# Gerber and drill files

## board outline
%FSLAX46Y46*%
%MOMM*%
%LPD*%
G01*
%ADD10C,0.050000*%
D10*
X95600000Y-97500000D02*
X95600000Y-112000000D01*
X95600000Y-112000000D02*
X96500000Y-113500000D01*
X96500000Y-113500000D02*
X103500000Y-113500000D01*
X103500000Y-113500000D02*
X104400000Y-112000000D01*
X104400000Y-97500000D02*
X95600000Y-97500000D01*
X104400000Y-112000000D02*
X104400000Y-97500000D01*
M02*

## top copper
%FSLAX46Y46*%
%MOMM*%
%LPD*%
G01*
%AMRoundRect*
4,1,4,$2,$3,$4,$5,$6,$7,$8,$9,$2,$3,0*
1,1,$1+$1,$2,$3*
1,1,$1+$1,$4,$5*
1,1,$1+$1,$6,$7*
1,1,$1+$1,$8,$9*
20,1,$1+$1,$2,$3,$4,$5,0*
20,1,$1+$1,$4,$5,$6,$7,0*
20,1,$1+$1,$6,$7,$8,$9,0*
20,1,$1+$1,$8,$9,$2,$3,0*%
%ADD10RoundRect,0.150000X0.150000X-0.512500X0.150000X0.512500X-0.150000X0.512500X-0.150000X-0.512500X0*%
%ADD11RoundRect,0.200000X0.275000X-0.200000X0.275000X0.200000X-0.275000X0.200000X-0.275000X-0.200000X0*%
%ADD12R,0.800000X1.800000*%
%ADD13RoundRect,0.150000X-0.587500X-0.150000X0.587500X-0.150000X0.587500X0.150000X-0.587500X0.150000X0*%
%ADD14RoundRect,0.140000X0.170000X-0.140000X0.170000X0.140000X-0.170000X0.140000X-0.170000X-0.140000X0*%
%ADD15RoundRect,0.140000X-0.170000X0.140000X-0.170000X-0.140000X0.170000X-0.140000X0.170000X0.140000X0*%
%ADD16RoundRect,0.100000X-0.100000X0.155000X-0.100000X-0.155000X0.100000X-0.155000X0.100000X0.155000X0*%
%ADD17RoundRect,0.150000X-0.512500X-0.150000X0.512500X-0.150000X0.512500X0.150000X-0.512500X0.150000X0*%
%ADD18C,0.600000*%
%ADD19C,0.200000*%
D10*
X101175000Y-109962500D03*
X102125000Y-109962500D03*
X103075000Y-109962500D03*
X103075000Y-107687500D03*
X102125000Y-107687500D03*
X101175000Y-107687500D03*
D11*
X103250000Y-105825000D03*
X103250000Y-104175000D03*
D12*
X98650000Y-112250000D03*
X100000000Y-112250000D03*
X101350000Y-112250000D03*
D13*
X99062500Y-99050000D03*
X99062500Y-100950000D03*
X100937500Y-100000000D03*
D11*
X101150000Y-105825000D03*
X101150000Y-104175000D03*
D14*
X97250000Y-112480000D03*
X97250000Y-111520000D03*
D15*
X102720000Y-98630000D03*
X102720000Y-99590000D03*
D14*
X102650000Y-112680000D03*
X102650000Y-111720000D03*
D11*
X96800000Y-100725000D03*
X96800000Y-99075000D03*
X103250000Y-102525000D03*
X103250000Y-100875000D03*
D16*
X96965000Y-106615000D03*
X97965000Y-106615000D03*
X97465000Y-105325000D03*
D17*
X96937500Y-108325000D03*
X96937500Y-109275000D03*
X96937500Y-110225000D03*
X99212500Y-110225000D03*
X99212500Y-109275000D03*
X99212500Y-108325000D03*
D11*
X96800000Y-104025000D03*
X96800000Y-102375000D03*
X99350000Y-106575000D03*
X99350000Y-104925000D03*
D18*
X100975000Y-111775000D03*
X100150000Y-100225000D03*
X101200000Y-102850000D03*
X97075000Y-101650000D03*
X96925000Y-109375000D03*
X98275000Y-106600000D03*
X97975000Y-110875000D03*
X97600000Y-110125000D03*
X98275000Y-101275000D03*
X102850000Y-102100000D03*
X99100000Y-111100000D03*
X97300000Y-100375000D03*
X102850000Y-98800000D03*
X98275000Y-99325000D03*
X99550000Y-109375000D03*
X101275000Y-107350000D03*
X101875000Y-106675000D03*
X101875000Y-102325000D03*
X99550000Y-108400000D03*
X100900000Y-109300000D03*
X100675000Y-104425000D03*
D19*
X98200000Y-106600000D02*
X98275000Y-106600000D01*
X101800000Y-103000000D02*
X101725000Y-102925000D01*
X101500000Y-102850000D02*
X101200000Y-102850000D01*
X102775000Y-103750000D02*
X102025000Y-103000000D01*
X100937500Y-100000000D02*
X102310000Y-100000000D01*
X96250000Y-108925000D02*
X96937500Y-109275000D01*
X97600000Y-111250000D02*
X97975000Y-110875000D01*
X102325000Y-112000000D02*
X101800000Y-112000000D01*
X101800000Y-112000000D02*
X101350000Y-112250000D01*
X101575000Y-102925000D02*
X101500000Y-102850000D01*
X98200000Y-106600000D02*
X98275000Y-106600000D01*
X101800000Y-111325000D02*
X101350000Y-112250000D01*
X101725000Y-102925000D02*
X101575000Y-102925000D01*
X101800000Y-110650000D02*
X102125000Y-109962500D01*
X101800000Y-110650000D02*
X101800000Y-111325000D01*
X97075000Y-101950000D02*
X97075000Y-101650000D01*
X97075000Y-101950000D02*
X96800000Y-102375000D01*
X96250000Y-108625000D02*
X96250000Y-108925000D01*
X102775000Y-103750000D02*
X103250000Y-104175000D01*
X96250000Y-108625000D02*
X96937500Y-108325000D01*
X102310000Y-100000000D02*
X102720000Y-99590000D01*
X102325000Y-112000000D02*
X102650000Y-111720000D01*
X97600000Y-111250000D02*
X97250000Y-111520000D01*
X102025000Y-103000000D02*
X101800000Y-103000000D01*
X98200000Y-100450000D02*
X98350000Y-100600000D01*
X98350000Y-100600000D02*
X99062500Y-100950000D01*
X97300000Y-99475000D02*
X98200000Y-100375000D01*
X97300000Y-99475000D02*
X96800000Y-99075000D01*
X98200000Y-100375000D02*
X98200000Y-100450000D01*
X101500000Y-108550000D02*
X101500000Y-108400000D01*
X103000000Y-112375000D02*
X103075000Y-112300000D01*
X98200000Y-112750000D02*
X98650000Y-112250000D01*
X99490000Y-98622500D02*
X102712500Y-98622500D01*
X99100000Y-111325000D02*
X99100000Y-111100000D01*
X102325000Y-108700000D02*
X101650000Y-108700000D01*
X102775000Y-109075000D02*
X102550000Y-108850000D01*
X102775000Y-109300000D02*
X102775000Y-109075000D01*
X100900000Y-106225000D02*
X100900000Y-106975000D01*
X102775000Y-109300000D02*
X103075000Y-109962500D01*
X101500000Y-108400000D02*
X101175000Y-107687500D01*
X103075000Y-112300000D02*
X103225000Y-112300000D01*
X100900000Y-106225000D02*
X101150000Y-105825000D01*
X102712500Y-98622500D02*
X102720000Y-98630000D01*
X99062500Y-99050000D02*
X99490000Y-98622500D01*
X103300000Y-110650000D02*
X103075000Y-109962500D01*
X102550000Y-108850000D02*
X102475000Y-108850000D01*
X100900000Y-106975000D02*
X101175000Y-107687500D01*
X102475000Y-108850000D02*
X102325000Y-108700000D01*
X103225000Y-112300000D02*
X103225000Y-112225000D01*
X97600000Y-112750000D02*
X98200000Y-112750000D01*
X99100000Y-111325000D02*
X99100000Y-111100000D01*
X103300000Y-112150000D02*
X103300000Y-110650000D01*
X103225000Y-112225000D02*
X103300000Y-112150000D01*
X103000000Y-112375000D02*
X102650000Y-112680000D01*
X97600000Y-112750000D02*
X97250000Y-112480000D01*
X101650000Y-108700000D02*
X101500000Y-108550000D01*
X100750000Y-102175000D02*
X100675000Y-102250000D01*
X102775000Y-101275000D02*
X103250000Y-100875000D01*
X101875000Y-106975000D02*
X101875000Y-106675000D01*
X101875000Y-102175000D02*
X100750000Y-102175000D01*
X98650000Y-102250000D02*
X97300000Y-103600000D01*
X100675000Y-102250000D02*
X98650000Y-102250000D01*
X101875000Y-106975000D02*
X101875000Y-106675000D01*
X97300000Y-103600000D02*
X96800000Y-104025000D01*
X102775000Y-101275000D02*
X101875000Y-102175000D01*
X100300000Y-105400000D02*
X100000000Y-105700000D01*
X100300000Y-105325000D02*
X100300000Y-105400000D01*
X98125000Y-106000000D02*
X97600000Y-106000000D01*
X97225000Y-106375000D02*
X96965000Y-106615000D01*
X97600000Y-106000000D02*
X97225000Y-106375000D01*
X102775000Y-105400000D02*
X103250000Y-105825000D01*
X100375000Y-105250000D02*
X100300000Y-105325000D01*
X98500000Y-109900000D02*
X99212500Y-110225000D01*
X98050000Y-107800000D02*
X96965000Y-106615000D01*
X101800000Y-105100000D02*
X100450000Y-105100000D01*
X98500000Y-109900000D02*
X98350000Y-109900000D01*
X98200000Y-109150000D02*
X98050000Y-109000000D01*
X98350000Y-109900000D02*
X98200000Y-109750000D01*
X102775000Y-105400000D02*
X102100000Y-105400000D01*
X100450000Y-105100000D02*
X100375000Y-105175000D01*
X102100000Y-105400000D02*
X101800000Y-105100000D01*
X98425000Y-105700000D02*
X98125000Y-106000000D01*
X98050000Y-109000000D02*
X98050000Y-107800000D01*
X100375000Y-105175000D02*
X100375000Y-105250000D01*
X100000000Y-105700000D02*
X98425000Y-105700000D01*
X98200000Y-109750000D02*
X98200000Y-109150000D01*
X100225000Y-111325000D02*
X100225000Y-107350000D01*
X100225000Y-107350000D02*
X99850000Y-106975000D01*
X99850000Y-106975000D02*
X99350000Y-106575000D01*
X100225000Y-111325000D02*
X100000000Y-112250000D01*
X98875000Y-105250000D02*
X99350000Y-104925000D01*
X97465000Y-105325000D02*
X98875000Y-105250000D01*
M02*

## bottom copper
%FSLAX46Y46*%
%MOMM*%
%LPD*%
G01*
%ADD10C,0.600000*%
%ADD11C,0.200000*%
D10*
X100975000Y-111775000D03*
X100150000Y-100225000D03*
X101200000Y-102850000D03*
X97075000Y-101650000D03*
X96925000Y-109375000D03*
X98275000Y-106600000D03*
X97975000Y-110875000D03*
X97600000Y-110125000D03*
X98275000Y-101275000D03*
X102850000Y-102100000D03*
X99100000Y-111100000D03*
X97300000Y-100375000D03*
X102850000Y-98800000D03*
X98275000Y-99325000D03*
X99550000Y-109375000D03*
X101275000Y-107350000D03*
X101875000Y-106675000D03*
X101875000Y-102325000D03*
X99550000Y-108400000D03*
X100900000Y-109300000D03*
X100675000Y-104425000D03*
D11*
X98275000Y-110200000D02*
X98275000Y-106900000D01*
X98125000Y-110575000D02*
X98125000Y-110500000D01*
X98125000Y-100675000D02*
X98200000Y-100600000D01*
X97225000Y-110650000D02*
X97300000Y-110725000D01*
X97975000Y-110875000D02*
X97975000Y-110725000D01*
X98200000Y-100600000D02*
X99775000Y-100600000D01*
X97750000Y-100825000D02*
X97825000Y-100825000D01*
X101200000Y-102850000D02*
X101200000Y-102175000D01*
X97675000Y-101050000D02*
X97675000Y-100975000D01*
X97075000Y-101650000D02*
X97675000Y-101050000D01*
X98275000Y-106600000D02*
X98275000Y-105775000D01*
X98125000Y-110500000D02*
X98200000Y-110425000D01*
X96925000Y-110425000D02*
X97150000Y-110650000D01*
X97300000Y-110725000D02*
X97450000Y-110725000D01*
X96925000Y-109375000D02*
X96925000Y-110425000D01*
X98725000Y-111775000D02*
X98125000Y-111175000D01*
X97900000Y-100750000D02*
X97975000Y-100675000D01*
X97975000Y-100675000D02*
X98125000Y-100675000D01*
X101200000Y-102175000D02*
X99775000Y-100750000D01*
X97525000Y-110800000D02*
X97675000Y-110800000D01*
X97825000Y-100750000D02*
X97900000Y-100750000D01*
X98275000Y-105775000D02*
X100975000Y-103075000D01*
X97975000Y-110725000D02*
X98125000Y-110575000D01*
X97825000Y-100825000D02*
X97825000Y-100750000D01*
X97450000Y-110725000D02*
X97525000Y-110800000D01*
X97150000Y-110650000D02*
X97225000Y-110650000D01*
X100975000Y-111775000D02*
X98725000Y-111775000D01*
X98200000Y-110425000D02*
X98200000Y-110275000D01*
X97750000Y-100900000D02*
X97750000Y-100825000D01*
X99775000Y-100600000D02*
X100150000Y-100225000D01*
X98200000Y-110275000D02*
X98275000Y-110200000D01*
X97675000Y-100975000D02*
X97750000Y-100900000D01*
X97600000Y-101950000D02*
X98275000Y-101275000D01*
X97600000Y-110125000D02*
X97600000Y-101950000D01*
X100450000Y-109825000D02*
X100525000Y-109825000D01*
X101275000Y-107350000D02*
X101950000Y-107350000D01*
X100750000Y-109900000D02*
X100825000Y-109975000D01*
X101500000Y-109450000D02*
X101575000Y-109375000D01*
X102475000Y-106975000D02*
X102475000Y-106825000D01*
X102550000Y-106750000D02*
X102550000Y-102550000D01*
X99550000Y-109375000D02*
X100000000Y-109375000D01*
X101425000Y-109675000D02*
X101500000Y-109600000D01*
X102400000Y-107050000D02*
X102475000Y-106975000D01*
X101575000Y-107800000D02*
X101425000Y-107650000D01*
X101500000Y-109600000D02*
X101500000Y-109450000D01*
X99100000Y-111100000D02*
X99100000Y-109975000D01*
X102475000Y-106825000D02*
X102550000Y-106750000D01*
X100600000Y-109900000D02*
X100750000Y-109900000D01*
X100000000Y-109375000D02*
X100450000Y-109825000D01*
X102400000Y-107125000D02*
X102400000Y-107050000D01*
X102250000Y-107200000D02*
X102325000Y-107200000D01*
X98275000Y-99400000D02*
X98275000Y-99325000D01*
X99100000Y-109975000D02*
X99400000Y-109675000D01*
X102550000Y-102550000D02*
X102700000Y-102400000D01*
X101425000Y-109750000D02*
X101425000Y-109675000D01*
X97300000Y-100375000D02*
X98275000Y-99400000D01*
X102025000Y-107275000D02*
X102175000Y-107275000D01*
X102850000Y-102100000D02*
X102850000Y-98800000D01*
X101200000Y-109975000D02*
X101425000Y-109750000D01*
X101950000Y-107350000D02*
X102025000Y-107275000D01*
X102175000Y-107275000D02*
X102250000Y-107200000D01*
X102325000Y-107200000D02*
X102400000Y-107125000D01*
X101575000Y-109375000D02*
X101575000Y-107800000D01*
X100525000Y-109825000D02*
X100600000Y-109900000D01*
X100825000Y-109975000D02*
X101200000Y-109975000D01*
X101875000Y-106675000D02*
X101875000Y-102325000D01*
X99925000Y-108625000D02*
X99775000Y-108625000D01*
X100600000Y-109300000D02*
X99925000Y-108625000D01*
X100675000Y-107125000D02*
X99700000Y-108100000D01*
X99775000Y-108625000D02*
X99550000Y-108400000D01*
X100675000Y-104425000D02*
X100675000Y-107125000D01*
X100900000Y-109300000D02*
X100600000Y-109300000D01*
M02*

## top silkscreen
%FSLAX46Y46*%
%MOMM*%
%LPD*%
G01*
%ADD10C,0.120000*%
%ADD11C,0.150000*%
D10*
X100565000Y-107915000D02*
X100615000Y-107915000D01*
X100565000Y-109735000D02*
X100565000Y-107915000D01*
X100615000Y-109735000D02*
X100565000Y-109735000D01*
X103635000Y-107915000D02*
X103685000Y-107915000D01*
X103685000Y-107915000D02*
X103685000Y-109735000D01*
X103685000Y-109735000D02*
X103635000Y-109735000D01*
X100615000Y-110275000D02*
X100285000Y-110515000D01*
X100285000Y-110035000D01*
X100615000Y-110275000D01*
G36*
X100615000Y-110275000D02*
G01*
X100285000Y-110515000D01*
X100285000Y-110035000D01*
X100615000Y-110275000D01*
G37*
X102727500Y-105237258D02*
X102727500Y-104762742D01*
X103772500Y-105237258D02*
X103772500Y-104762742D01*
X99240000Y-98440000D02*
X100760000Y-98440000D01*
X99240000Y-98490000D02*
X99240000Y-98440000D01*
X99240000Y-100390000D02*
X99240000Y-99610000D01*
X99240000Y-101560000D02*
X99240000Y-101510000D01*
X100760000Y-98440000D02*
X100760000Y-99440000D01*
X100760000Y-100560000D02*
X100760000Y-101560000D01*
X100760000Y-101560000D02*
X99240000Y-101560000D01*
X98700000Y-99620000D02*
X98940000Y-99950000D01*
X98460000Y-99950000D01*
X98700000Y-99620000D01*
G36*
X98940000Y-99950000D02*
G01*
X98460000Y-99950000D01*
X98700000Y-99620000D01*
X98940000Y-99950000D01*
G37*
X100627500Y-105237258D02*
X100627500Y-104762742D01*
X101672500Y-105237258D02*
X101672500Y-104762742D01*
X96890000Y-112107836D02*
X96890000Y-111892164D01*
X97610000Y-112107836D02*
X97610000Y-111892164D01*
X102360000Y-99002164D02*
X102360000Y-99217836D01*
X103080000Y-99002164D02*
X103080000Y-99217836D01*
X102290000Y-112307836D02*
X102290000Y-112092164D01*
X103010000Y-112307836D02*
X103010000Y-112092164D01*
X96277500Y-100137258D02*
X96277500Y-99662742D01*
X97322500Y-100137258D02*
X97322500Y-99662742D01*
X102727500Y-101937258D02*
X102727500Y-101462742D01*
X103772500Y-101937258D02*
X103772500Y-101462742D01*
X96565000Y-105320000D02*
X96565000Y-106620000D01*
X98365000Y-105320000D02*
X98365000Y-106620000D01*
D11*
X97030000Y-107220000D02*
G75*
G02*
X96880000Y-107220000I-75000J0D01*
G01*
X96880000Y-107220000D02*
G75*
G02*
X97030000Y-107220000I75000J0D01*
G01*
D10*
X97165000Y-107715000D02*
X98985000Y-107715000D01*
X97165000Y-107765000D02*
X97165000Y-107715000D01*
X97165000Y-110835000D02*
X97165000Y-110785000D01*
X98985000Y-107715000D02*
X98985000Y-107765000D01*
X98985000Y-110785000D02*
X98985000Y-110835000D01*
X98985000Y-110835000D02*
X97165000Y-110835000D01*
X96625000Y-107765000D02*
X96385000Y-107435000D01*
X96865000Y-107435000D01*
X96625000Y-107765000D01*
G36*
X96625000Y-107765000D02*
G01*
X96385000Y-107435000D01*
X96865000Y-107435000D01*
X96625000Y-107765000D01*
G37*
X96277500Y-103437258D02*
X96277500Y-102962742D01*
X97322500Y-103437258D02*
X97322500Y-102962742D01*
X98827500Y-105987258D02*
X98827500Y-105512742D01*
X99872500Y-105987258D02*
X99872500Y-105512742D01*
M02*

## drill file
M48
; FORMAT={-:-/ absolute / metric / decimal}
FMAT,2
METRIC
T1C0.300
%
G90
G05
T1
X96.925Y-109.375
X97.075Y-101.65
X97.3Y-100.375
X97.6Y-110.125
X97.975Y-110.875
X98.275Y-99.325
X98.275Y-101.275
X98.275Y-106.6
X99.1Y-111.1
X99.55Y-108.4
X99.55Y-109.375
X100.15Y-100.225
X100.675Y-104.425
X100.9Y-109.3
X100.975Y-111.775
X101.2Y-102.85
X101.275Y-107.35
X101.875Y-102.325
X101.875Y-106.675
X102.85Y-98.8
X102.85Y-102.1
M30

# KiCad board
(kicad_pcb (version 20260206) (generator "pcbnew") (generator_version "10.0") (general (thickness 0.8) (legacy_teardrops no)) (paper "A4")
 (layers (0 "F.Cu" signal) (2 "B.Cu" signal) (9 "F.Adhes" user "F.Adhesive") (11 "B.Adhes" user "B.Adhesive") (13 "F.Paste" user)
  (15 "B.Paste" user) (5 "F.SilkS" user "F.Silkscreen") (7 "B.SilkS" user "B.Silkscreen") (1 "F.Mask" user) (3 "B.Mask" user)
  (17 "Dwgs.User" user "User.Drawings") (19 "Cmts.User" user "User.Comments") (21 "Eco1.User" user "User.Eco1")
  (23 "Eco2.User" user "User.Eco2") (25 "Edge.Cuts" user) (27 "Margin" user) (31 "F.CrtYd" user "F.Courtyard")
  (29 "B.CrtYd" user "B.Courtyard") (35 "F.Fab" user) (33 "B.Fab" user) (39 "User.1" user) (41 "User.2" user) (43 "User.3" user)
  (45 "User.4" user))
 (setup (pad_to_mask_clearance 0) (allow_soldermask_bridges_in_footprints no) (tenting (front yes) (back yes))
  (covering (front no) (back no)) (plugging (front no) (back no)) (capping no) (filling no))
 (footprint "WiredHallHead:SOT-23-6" (layer "F.Cu") (at 102.125 108.825 90)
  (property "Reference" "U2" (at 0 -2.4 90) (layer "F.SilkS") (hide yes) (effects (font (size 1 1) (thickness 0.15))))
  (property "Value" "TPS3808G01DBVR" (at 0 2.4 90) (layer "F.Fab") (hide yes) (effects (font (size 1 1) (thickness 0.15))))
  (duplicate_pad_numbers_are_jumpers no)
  (fp_line (start 0.91 -1.56) (end 0.91 -1.51) (stroke (width 0.12) (type solid)) (layer "F.SilkS"))
  (fp_line (start -0.91 -1.56) (end 0.91 -1.56) (stroke (width 0.12) (type solid)) (layer "F.SilkS"))
  (fp_line (start -0.91 -1.51) (end -0.91 -1.56) (stroke (width 0.12) (type solid)) (layer "F.SilkS"))
  (fp_line (start 0.91 1.51) (end 0.91 1.56) (stroke (width 0.12) (type solid)) (layer "F.SilkS"))
  (fp_line (start 0.91 1.56) (end -0.91 1.56) (stroke (width 0.12) (type solid)) (layer "F.SilkS"))
  (fp_line (start -0.91 1.56) (end -0.91 1.51) (stroke (width 0.12) (type solid)) (layer "F.SilkS"))
  (fp_poly (pts (xy -1.45 -1.51) (xy -1.69 -1.84) (xy -1.21 -1.84)) (stroke (width 0.12) (type solid)) (fill yes) (layer "F.SilkS"))
  (pad "1" smd roundrect (at -1.1375 -0.95 90) (size 1.325 0.6) (layers "F.Cu" "F.Mask" "F.Paste") (roundrect_rratio 0.25)
   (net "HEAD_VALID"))
  (pad "2" smd roundrect (at -1.1375 0 90) (size 1.325 0.6) (layers "F.Cu" "F.Mask" "F.Paste") (roundrect_rratio 0.25) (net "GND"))
  (pad "3" smd roundrect (at -1.1375 0.95 90) (size 1.325 0.6) (layers "F.Cu" "F.Mask" "F.Paste") (roundrect_rratio 0.25) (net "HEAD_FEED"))
  (pad "4" smd roundrect (at 1.1375 0.95 90) (size 1.325 0.6) (layers "F.Cu" "F.Mask" "F.Paste") (roundrect_rratio 0.25)
   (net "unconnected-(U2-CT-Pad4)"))
  (pad "5" smd roundrect (at 1.1375 0 90) (size 1.325 0.6) (layers "F.Cu" "F.Mask" "F.Paste") (roundrect_rratio 0.25) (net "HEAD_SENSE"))
  (pad "6" smd roundrect (at 1.1375 -0.95 90) (size 1.325 0.6) (layers "F.Cu" "F.Mask" "F.Paste") (roundrect_rratio 0.25) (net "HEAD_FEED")))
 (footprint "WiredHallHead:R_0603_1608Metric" (layer "F.Cu") (at 103.25 105 90)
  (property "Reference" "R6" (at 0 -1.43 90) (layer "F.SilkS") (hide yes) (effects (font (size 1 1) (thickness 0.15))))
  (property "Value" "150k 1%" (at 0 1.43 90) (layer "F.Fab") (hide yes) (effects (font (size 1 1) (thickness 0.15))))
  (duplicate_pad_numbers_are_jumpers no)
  (fp_line (start -0.237258 -0.5225) (end 0.237258 -0.5225) (stroke (width 0.12) (type solid)) (layer "F.SilkS"))
  (fp_line (start -0.237258 0.5225) (end 0.237258 0.5225) (stroke (width 0.12) (type solid)) (layer "F.SilkS"))
  (pad "1" smd roundrect (at -0.825 0 90) (size 0.8 0.95) (layers "F.Cu" "F.Mask" "F.Paste") (roundrect_rratio 0.25) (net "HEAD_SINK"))
  (pad "2" smd roundrect (at 0.825 0 90) (size 0.8 0.95) (layers "F.Cu" "F.Mask" "F.Paste") (roundrect_rratio 0.25) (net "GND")))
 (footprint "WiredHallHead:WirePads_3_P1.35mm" (layer "F.Cu") (at 100 112.25)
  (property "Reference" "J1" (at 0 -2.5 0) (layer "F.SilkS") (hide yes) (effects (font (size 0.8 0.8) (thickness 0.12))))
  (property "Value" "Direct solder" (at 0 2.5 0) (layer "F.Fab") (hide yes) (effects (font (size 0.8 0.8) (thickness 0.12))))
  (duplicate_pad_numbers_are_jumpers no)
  (pad "1" smd rect (at -1.35 0) (size 0.8 1.8) (layers "F.Cu" "F.Mask") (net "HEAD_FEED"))
  (pad "2" smd rect (at 0 0) (size 0.8 1.8) (layers "F.Cu" "F.Mask") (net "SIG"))
  (pad "3" smd rect (at 1.35 0) (size 0.8 1.8) (layers "F.Cu" "F.Mask") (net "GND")))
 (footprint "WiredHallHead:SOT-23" (layer "F.Cu") (at 100 100)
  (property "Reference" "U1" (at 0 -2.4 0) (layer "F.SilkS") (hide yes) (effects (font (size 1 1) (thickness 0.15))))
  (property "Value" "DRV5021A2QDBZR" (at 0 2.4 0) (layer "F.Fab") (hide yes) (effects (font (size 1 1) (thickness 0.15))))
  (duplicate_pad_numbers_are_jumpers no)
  (fp_line (start -0.76 -1.56) (end 0.76 -1.56) (stroke (width 0.12) (type solid)) (layer "F.SilkS"))
  (fp_line (start -0.76 -1.51) (end -0.76 -1.56) (stroke (width 0.12) (type solid)) (layer "F.SilkS"))
  (fp_line (start -0.76 0.39) (end -0.76 -0.39) (stroke (width 0.12) (type solid)) (layer "F.SilkS"))
  (fp_line (start -0.76 1.56) (end -0.76 1.51) (stroke (width 0.12) (type solid)) (layer "F.SilkS"))
  (fp_line (start 0.76 -1.56) (end 0.76 -0.56) (stroke (width 0.12) (type solid)) (layer "F.SilkS"))
  (fp_line (start 0.76 0.56) (end 0.76 1.56) (stroke (width 0.12) (type solid)) (layer "F.SilkS"))
  (fp_line (start 0.76 1.56) (end -0.76 1.56) (stroke (width 0.12) (type solid)) (layer "F.SilkS"))
  (fp_poly (pts (xy -1.3 -0.38) (xy -1.06 -0.05) (xy -1.54 -0.05)) (stroke (width 0.12) (type solid)) (fill yes) (layer "F.SilkS"))
  (pad "1" smd roundrect (at -0.9375 -0.95) (size 1.475 0.6) (layers "F.Cu" "F.Mask" "F.Paste") (roundrect_rratio 0.25) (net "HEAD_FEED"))
  (pad "2" smd roundrect (at -0.9375 0.95) (size 1.475 0.6) (layers "F.Cu" "F.Mask" "F.Paste") (roundrect_rratio 0.25) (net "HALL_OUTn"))
  (pad "3" smd roundrect (at 0.9375 0) (size 1.475 0.6) (layers "F.Cu" "F.Mask" "F.Paste") (roundrect_rratio 0.25) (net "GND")))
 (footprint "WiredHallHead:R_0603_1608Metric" (layer "F.Cu") (at 101.15 105 90)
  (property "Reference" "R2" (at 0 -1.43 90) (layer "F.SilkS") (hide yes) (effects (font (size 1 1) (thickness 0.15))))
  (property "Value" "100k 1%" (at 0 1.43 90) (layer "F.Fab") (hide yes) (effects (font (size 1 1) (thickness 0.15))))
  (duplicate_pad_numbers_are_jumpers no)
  (fp_line (start -0.237258 -0.5225) (end 0.237258 -0.5225) (stroke (width 0.12) (type solid)) (layer "F.SilkS"))
  (fp_line (start -0.237258 0.5225) (end 0.237258 0.5225) (stroke (width 0.12) (type solid)) (layer "F.SilkS"))
  (pad "1" smd roundrect (at -0.825 0 90) (size 0.8 0.95) (layers "F.Cu" "F.Mask" "F.Paste") (roundrect_rratio 0.25) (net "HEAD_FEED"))
  (pad "2" smd roundrect (at 0.825 0 90) (size 0.8 0.95) (layers "F.Cu" "F.Mask" "F.Paste") (roundrect_rratio 0.25) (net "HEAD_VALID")))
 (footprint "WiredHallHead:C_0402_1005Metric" (layer "F.Cu") (at 97.25 112 90)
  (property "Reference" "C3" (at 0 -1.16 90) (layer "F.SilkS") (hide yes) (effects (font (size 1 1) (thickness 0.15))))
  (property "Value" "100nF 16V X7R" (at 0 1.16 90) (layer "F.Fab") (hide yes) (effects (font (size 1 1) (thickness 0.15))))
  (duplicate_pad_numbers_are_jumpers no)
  (fp_line (start -0.107836 -0.36) (end 0.107836 -0.36) (stroke (width 0.12) (type solid)) (layer "F.SilkS"))
  (fp_line (start -0.107836 0.36) (end 0.107836 0.36) (stroke (width 0.12) (type solid)) (layer "F.SilkS"))
  (pad "1" smd roundrect (at -0.48 0 90) (size 0.56 0.62) (layers "F.Cu" "F.Mask" "F.Paste") (roundrect_rratio 0.25) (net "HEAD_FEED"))
  (pad "2" smd roundrect (at 0.48 0 90) (size 0.56 0.62) (layers "F.Cu" "F.Mask" "F.Paste") (roundrect_rratio 0.25) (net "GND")))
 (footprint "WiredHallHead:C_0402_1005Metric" (layer "F.Cu") (at 102.72 99.11 -90)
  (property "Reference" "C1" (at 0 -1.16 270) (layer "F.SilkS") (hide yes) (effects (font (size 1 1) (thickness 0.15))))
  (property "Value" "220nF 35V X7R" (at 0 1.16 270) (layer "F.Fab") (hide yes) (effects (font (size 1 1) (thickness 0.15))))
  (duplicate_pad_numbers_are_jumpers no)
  (fp_line (start -0.107836 0.36) (end 0.107836 0.36) (stroke (width 0.12) (type solid)) (layer "F.SilkS"))
  (fp_line (start -0.107836 -0.36) (end 0.107836 -0.36) (stroke (width 0.12) (type solid)) (layer "F.SilkS"))
  (pad "1" smd roundrect (at -0.48 0 270) (size 0.56 0.62) (layers "F.Cu" "F.Mask" "F.Paste") (roundrect_rratio 0.25) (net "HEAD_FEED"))
  (pad "2" smd roundrect (at 0.48 0 270) (size 0.56 0.62) (layers "F.Cu" "F.Mask" "F.Paste") (roundrect_rratio 0.25) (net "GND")))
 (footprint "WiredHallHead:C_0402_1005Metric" (layer "F.Cu") (at 102.65 112.2 90)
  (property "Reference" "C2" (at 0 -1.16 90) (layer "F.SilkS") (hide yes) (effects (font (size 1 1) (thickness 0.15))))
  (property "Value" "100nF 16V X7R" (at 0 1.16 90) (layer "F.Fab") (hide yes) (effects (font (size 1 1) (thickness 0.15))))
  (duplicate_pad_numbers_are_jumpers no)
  (fp_line (start -0.107836 -0.36) (end 0.107836 -0.36) (stroke (width 0.12) (type solid)) (layer "F.SilkS"))
  (fp_line (start -0.107836 0.36) (end 0.107836 0.36) (stroke (width 0.12) (type solid)) (layer "F.SilkS"))
  (pad "1" smd roundrect (at -0.48 0 90) (size 0.56 0.62) (layers "F.Cu" "F.Mask" "F.Paste") (roundrect_rratio 0.25) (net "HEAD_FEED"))
  (pad "2" smd roundrect (at 0.48 0 90) (size 0.56 0.62) (layers "F.Cu" "F.Mask" "F.Paste") (roundrect_rratio 0.25) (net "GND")))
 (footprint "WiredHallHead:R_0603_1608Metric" (layer "F.Cu") (at 96.8 99.9 90)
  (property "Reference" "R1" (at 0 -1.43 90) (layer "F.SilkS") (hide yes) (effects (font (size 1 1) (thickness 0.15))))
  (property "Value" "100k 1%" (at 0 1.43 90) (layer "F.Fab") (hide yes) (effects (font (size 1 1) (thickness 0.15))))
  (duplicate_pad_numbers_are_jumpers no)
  (fp_line (start -0.237258 -0.5225) (end 0.237258 -0.5225) (stroke (width 0.12) (type solid)) (layer "F.SilkS"))
  (fp_line (start -0.237258 0.5225) (end 0.237258 0.5225) (stroke (width 0.12) (type solid)) (layer "F.SilkS"))
  (pad "1" smd roundrect (at -0.825 0 90) (size 0.8 0.95) (layers "F.Cu" "F.Mask" "F.Paste") (roundrect_rratio 0.25) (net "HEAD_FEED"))
  (pad "2" smd roundrect (at 0.825 0 90) (size 0.8 0.95) (layers "F.Cu" "F.Mask" "F.Paste") (roundrect_rratio 0.25) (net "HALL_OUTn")))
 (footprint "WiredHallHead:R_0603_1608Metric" (layer "F.Cu") (at 103.25 101.7 90)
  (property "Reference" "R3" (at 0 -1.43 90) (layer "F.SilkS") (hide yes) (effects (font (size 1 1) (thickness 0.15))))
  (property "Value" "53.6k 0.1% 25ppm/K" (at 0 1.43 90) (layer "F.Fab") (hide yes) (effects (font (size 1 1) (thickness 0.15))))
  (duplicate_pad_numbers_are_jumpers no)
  (fp_line (start -0.237258 -0.5225) (end 0.237258 -0.5225) (stroke (width 0.12) (type solid)) (layer "F.SilkS"))
  (fp_line (start -0.237258 0.5225) (end 0.237258 0.5225) (stroke (width 0.12) (type solid)) (layer "F.SilkS"))
  (pad "1" smd roundrect (at -0.825 0 90) (size 0.8 0.95) (layers "F.Cu" "F.Mask" "F.Paste") (roundrect_rratio 0.25) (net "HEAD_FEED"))
  (pad "2" smd roundrect (at 0.825 0 90) (size 0.8 0.95) (layers "F.Cu" "F.Mask" "F.Paste") (roundrect_rratio 0.25) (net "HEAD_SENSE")))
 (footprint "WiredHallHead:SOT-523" (layer "F.Cu") (at 97.465 105.97 90)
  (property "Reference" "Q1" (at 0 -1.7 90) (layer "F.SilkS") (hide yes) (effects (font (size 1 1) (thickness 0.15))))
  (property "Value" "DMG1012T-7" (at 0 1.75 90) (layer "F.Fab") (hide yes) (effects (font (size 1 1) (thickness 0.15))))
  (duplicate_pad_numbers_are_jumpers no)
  (fp_line (start 0.65 -0.9) (end -0.65 -0.9) (stroke (width 0.12) (type solid)) (layer "F.SilkS"))
  (fp_line (start 0.65 0.9) (end -0.65 0.9) (stroke (width 0.12) (type solid)) (layer "F.SilkS"))
  (fp_circle (center -1.25 -0.51) (end -1.1 -0.51) (stroke (width 0) (type solid)) (fill yes) (layer "F.SilkS"))
  (pad "1" smd roundrect (at -0.645 -0.5 270) (size 0.51 0.4) (layers "F.Cu" "F.Mask" "F.Paste") (roundrect_rratio 0.25) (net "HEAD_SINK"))
  (pad "2" smd roundrect (at -0.645 0.5 270) (size 0.51 0.4) (layers "F.Cu" "F.Mask" "F.Paste") (roundrect_rratio 0.25) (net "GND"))
  (pad "3" smd roundrect (at 0.645 0 270) (size 0.51 0.4) (layers "F.Cu" "F.Mask" "F.Paste") (roundrect_rratio 0.25) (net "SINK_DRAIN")))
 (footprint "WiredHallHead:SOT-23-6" (layer "F.Cu") (at 98.075 109.275)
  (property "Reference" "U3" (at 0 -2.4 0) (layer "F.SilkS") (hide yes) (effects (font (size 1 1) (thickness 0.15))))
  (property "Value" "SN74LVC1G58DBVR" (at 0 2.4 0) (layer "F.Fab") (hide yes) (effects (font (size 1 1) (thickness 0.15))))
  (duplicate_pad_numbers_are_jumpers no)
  (fp_line (start -0.91 -1.56) (end 0.91 -1.56) (stroke (width 0.12) (type solid)) (layer "F.SilkS"))
  (fp_line (start -0.91 -1.51) (end -0.91 -1.56) (stroke (width 0.12) (type solid)) (layer "F.SilkS"))
  (fp_line (start -0.91 1.56) (end -0.91 1.51) (stroke (width 0.12) (type solid)) (layer "F.SilkS"))
  (fp_line (start 0.91 -1.56) (end 0.91 -1.51) (stroke (width 0.12) (type solid)) (layer "F.SilkS"))
  (fp_line (start 0.91 1.51) (end 0.91 1.56) (stroke (width 0.12) (type solid)) (layer "F.SilkS"))
  (fp_line (start 0.91 1.56) (end -0.91 1.56) (stroke (width 0.12) (type solid)) (layer "F.SilkS"))
  (fp_poly (pts (xy -1.45 -1.51) (xy -1.69 -1.84) (xy -1.21 -1.84)) (stroke (width 0.12) (type solid)) (fill yes) (layer "F.SilkS"))
  (pad "1" smd roundrect (at -1.1375 -0.95) (size 1.325 0.6) (layers "F.Cu" "F.Mask" "F.Paste") (roundrect_rratio 0.25) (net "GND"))
  (pad "2" smd roundrect (at -1.1375 0) (size 1.325 0.6) (layers "F.Cu" "F.Mask" "F.Paste") (roundrect_rratio 0.25) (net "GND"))
  (pad "3" smd roundrect (at -1.1375 0.95) (size 1.325 0.6) (layers "F.Cu" "F.Mask" "F.Paste") (roundrect_rratio 0.25) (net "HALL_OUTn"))
  (pad "4" smd roundrect (at 1.1375 0.95) (size 1.325 0.6) (layers "F.Cu" "F.Mask" "F.Paste") (roundrect_rratio 0.25) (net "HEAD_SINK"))
  (pad "5" smd roundrect (at 1.1375 0) (size 1.325 0.6) (layers "F.Cu" "F.Mask" "F.Paste") (roundrect_rratio 0.25) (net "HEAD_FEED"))
  (pad "6" smd roundrect (at 1.1375 -0.95) (size 1.325 0.6) (layers "F.Cu" "F.Mask" "F.Paste") (roundrect_rratio 0.25) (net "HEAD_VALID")))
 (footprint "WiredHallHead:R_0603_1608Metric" (layer "F.Cu") (at 96.8 103.2 90)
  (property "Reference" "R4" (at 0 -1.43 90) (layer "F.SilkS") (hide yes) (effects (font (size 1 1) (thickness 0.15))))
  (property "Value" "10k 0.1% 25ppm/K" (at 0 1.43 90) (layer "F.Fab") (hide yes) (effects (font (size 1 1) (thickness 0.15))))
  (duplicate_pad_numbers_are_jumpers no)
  (fp_line (start -0.237258 -0.5225) (end 0.237258 -0.5225) (stroke (width 0.12) (type solid)) (layer "F.SilkS"))
  (fp_line (start -0.237258 0.5225) (end 0.237258 0.5225) (stroke (width 0.12) (type solid)) (layer "F.SilkS"))
  (pad "1" smd roundrect (at -0.825 0 90) (size 0.8 0.95) (layers "F.Cu" "F.Mask" "F.Paste") (roundrect_rratio 0.25) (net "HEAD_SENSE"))
  (pad "2" smd roundrect (at 0.825 0 90) (size 0.8 0.95) (layers "F.Cu" "F.Mask" "F.Paste") (roundrect_rratio 0.25) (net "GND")))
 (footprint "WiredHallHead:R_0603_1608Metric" (layer "F.Cu") (at 99.35 105.75 90)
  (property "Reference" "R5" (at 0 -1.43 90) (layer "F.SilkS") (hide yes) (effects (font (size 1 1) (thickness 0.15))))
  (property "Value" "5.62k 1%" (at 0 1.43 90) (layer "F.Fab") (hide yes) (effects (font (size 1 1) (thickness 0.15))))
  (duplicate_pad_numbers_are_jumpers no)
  (fp_line (start -0.237258 -0.5225) (end 0.237258 -0.5225) (stroke (width 0.12) (type solid)) (layer "F.SilkS"))
  (fp_line (start -0.237258 0.5225) (end 0.237258 0.5225) (stroke (width 0.12) (type solid)) (layer "F.SilkS"))
  (pad "1" smd roundrect (at -0.825 0 90) (size 0.8 0.95) (layers "F.Cu" "F.Mask" "F.Paste") (roundrect_rratio 0.25) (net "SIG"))
  (pad "2" smd roundrect (at 0.825 0 90) (size 0.8 0.95) (layers "F.Cu" "F.Mask" "F.Paste") (roundrect_rratio 0.25) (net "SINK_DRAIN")))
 (gr_line (start 95.6 97.5) (end 95.6 112) (stroke (width 0.05) (type default)) (layer "Edge.Cuts"))
 (gr_line (start 95.6 112) (end 96.5 113.5) (stroke (width 0.05) (type default)) (layer "Edge.Cuts"))
 (gr_line (start 96.5 113.5) (end 103.5 113.5) (stroke (width 0.05) (type default)) (layer "Edge.Cuts"))
 (gr_line (start 103.5 113.5) (end 104.4 112) (stroke (width 0.05) (type default)) (layer "Edge.Cuts"))
 (gr_line (start 104.4 97.5) (end 95.6 97.5) (stroke (width 0.05) (type default)) (layer "Edge.Cuts"))
 (gr_line (start 104.4 112) (end 104.4 97.5) (stroke (width 0.05) (type default)) (layer "Edge.Cuts"))
 (segment (start 98.2 106.6) (end 98.275 106.6) (width 0.2) (layer "F.Cu") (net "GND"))
 (segment (start 101.8 103) (end 101.725 102.925) (width 0.2) (layer "F.Cu") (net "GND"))
 (segment (start 101.5 102.85) (end 101.2 102.85) (width 0.2) (layer "F.Cu") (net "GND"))
 (segment (start 102.775 103.75) (end 102.025 103) (width 0.2) (layer "F.Cu") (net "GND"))
 (segment (start 100.9375 100) (end 102.31 100) (width 0.2) (layer "F.Cu") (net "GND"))
 (segment (start 96.25 108.925) (end 96.9375 109.275) (width 0.2) (layer "F.Cu") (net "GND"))
 (segment (start 97.6 111.25) (end 97.975 110.875) (width 0.2) (layer "F.Cu") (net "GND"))
 (segment (start 102.325 112) (end 101.8 112) (width 0.2) (layer "F.Cu") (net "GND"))
 (segment (start 101.8 112) (end 101.35 112.25) (width 0.2) (layer "F.Cu") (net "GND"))
 (segment (start 101.575 102.925) (end 101.5 102.85) (width 0.2) (layer "F.Cu") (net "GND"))
 (segment (start 98.2 106.6) (end 98.275 106.6) (width 0.2) (layer "F.Cu") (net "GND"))
 (segment (start 101.8 111.325) (end 101.35 112.25) (width 0.2) (layer "F.Cu") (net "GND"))
 (segment (start 101.725 102.925) (end 101.575 102.925) (width 0.2) (layer "F.Cu") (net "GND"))
 (segment (start 101.8 110.65) (end 102.125 109.9625) (width 0.2) (layer "F.Cu") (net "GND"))
 (segment (start 101.8 110.65) (end 101.8 111.325) (width 0.2) (layer "F.Cu") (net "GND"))
 (segment (start 97.075 101.95) (end 97.075 101.65) (width 0.2) (layer "F.Cu") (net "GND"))
 (segment (start 97.075 101.95) (end 96.8 102.375) (width 0.2) (layer "F.Cu") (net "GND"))
 (segment (start 96.25 108.625) (end 96.25 108.925) (width 0.2) (layer "F.Cu") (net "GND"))
 (segment (start 102.775 103.75) (end 103.25 104.175) (width 0.2) (layer "F.Cu") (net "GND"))
 (segment (start 96.25 108.625) (end 96.9375 108.325) (width 0.2) (layer "F.Cu") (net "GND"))
 (segment (start 102.31 100) (end 102.72 99.59) (width 0.2) (layer "F.Cu") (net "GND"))
 (segment (start 102.325 112) (end 102.65 111.72) (width 0.2) (layer "F.Cu") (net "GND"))
 (segment (start 97.6 111.25) (end 97.25 111.52) (width 0.2) (layer "F.Cu") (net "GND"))
 (segment (start 102.025 103) (end 101.8 103) (width 0.2) (layer "F.Cu") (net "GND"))
 (via (at 100.975 111.775) (size 0.6) (drill 0.3) (layers "F.Cu" "B.Cu") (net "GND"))
 (via (at 100.15 100.225) (size 0.6) (drill 0.3) (layers "F.Cu" "B.Cu") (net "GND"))
 (via (at 101.2 102.85) (size 0.6) (drill 0.3) (layers "F.Cu" "B.Cu") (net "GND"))
 (via (at 97.075 101.65) (size 0.6) (drill 0.3) (layers "F.Cu" "B.Cu") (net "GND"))
 (via (at 96.925 109.375) (size 0.6) (drill 0.3) (layers "F.Cu" "B.Cu") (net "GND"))
 (via (at 98.275 106.6) (size 0.6) (drill 0.3) (layers "F.Cu" "B.Cu") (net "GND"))
 (via (at 97.975 110.875) (size 0.6) (drill 0.3) (layers "F.Cu" "B.Cu") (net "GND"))
 (segment (start 98.275 110.2) (end 98.275 106.9) (width 0.2) (layer "B.Cu") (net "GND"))
 (segment (start 98.125 110.575) (end 98.125 110.5) (width 0.2) (layer "B.Cu") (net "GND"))
 (segment (start 98.125 100.675) (end 98.2 100.6) (width 0.2) (layer "B.Cu") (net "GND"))
 (segment (start 97.225 110.65) (end 97.3 110.725) (width 0.2) (layer "B.Cu") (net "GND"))
 (segment (start 97.975 110.875) (end 97.975 110.725) (width 0.2) (layer "B.Cu") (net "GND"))
 (segment (start 98.2 100.6) (end 99.775 100.6) (width 0.2) (layer "B.Cu") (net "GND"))
 (segment (start 97.75 100.825) (end 97.825 100.825) (width 0.2) (layer "B.Cu") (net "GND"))
 (segment (start 101.2 102.85) (end 101.2 102.175) (width 0.2) (layer "B.Cu") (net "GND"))
 (segment (start 97.675 101.05) (end 97.675 100.975) (width 0.2) (layer "B.Cu") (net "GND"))
 (segment (start 97.075 101.65) (end 97.675 101.05) (width 0.2) (layer "B.Cu") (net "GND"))
 (segment (start 98.275 106.6) (end 98.275 105.775) (width 0.2) (layer "B.Cu") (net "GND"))
 (segment (start 98.125 110.5) (end 98.2 110.425) (width 0.2) (layer "B.Cu") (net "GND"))
 (segment (start 96.925 110.425) (end 97.15 110.65) (width 0.2) (layer "B.Cu") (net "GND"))
 (segment (start 97.3 110.725) (end 97.45 110.725) (width 0.2) (layer "B.Cu") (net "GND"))
 (segment (start 96.925 109.375) (end 96.925 110.425) (width 0.2) (layer "B.Cu") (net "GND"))
 (segment (start 98.725 111.775) (end 98.125 111.175) (width 0.2) (layer "B.Cu") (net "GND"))
 (segment (start 97.9 100.75) (end 97.975 100.675) (width 0.2) (layer "B.Cu") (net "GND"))
 (segment (start 97.975 100.675) (end 98.125 100.675) (width 0.2) (layer "B.Cu") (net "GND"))
 (segment (start 101.2 102.175) (end 99.775 100.75) (width 0.2) (layer "B.Cu") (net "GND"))
 (segment (start 97.525 110.8) (end 97.675 110.8) (width 0.2) (layer "B.Cu") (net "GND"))
 (segment (start 97.825 100.75) (end 97.9 100.75) (width 0.2) (layer "B.Cu") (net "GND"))
 (segment (start 98.275 105.775) (end 100.975 103.075) (width 0.2) (layer "B.Cu") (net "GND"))
 (segment (start 97.975 110.725) (end 98.125 110.575) (width 0.2) (layer "B.Cu") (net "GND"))
 (segment (start 97.825 100.825) (end 97.825 100.75) (width 0.2) (layer "B.Cu") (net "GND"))
 (segment (start 97.45 110.725) (end 97.525 110.8) (width 0.2) (layer "B.Cu") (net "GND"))
 (segment (start 97.15 110.65) (end 97.225 110.65) (width 0.2) (layer "B.Cu") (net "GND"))
 (segment (start 100.975 111.775) (end 98.725 111.775) (width 0.2) (layer "B.Cu") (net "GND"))
 (segment (start 98.2 110.425) (end 98.2 110.275) (width 0.2) (layer "B.Cu") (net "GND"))
 (segment (start 97.75 100.9) (end 97.75 100.825) (width 0.2) (layer "B.Cu") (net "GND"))
 (segment (start 99.775 100.6) (end 100.15 100.225) (width 0.2) (layer "B.Cu") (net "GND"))
 (segment (start 98.2 110.275) (end 98.275 110.2) (width 0.2) (layer "B.Cu") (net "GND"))
 (segment (start 97.675 100.975) (end 97.75 100.9) (width 0.2) (layer "B.Cu") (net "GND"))
 (segment (start 98.2 100.45) (end 98.35 100.6) (width 0.2) (layer "F.Cu") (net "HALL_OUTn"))
 (segment (start 98.35 100.6) (end 99.0625 100.95) (width 0.2) (layer "F.Cu") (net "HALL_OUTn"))
 (segment (start 97.3 99.475) (end 98.2 100.375) (width 0.2) (layer "F.Cu") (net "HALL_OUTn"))
 (segment (start 97.3 99.475) (end 96.8 99.075) (width 0.2) (layer "F.Cu") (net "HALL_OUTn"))
 (segment (start 98.2 100.375) (end 98.2 100.45) (width 0.2) (layer "F.Cu") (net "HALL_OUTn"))
 (via (at 97.6 110.125) (size 0.6) (drill 0.3) (layers "F.Cu" "B.Cu") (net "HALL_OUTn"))
 (via (at 98.275 101.275) (size 0.6) (drill 0.3) (layers "F.Cu" "B.Cu") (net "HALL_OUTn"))
 (segment (start 97.6 101.95) (end 98.275 101.275) (width 0.2) (layer "B.Cu") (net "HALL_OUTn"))
 (segment (start 97.6 110.125) (end 97.6 101.95) (width 0.2) (layer "B.Cu") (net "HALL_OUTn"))
 (segment (start 101.5 108.55) (end 101.5 108.4) (width 0.2) (layer "F.Cu") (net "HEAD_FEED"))
 (segment (start 103 112.375) (end 103.075 112.3) (width 0.2) (layer "F.Cu") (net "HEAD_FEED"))
 (segment (start 98.2 112.75) (end 98.65 112.25) (width 0.2) (layer "F.Cu") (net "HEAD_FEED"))
 (segment (start 99.49 98.6225) (end 102.7125 98.6225) (width 0.2) (layer "F.Cu") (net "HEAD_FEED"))
 (segment (start 99.1 111.325) (end 99.1 111.1) (width 0.2) (layer "F.Cu") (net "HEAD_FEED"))
 (segment (start 102.325 108.7) (end 101.65 108.7) (width 0.2) (layer "F.Cu") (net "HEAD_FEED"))
 (segment (start 102.775 109.075) (end 102.55 108.85) (width 0.2) (layer "F.Cu") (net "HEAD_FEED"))
 (segment (start 102.775 109.3) (end 102.775 109.075) (width 0.2) (layer "F.Cu") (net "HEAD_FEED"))
 (segment (start 100.9 106.225) (end 100.9 106.975) (width 0.2) (layer "F.Cu") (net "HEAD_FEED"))
 (segment (start 102.775 109.3) (end 103.075 109.9625) (width 0.2) (layer "F.Cu") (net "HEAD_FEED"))
 (segment (start 101.5 108.4) (end 101.175 107.6875) (width 0.2) (layer "F.Cu") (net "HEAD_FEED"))
 (segment (start 103.075 112.3) (end 103.225 112.3) (width 0.2) (layer "F.Cu") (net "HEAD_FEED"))
 (segment (start 100.9 106.225) (end 101.15 105.825) (width 0.2) (layer "F.Cu") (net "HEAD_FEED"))
 (segment (start 102.7125 98.6225) (end 102.72 98.63) (width 0.2) (layer "F.Cu") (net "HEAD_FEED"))
 (segment (start 99.0625 99.05) (end 99.49 98.6225) (width 0.2) (layer "F.Cu") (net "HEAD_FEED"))
 (segment (start 103.3 110.65) (end 103.075 109.9625) (width 0.2) (layer "F.Cu") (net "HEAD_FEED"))
 (segment (start 102.55 108.85) (end 102.475 108.85) (width 0.2) (layer "F.Cu") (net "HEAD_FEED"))
 (segment (start 100.9 106.975) (end 101.175 107.6875) (width 0.2) (layer "F.Cu") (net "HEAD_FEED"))
 (segment (start 102.475 108.85) (end 102.325 108.7) (width 0.2) (layer "F.Cu") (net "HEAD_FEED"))
 (segment (start 103.225 112.3) (end 103.225 112.225) (width 0.2) (layer "F.Cu") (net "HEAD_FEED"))
 (segment (start 97.6 112.75) (end 98.2 112.75) (width 0.2) (layer "F.Cu") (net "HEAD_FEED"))
 (segment (start 99.1 111.325) (end 99.1 111.1) (width 0.2) (layer "F.Cu") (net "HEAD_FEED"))
 (segment (start 103.3 112.15) (end 103.3 110.65) (width 0.2) (layer "F.Cu") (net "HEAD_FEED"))
 (segment (start 103.225 112.225) (end 103.3 112.15) (width 0.2) (layer "F.Cu") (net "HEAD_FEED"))
 (segment (start 103 112.375) (end 102.65 112.68) (width 0.2) (layer "F.Cu") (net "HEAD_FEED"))
 (segment (start 97.6 112.75) (end 97.25 112.48) (width 0.2) (layer "F.Cu") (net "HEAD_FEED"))
 (segment (start 101.65 108.7) (end 101.5 108.55) (width 0.2) (layer "F.Cu") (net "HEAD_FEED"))
 (via (at 102.85 102.1) (size 0.6) (drill 0.3) (layers "F.Cu" "B.Cu") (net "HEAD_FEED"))
 (via (at 99.1 111.1) (size 0.6) (drill 0.3) (layers "F.Cu" "B.Cu") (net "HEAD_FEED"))
 (via (at 97.3 100.375) (size 0.6) (drill 0.3) (layers "F.Cu" "B.Cu") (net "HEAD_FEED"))
 (via (at 102.85 98.8) (size 0.6) (drill 0.3) (layers "F.Cu" "B.Cu") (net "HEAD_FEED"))
 (via (at 98.275 99.325) (size 0.6) (drill 0.3) (layers "F.Cu" "B.Cu") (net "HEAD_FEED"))
 (via (at 99.55 109.375) (size 0.6) (drill 0.3) (layers "F.Cu" "B.Cu") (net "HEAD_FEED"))
 (via (at 101.275 107.35) (size 0.6) (drill 0.3) (layers "F.Cu" "B.Cu") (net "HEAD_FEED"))
 (segment (start 100.45 109.825) (end 100.525 109.825) (width 0.2) (layer "B.Cu") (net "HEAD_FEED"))
 (segment (start 101.275 107.35) (end 101.95 107.35) (width 0.2) (layer "B.Cu") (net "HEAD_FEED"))
 (segment (start 100.75 109.9) (end 100.825 109.975) (width 0.2) (layer "B.Cu") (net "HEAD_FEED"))
 (segment (start 101.5 109.45) (end 101.575 109.375) (width 0.2) (layer "B.Cu") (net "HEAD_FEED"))
 (segment (start 102.475 106.975) (end 102.475 106.825) (width 0.2) (layer "B.Cu") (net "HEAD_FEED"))
 (segment (start 102.55 106.75) (end 102.55 102.55) (width 0.2) (layer "B.Cu") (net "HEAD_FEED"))
 (segment (start 99.55 109.375) (end 100 109.375) (width 0.2) (layer "B.Cu") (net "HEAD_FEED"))
 (segment (start 101.425 109.675) (end 101.5 109.6) (width 0.2) (layer "B.Cu") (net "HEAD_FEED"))
 (segment (start 102.4 107.05) (end 102.475 106.975) (width 0.2) (layer "B.Cu") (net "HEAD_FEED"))
 (segment (start 101.575 107.8) (end 101.425 107.65) (width 0.2) (layer "B.Cu") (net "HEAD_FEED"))
 (segment (start 101.5 109.6) (end 101.5 109.45) (width 0.2) (layer "B.Cu") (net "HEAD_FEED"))
 (segment (start 99.1 111.1) (end 99.1 109.975) (width 0.2) (layer "B.Cu") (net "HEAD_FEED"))
 (segment (start 102.475 106.825) (end 102.55 106.75) (width 0.2) (layer "B.Cu") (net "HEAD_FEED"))
 (segment (start 100.6 109.9) (end 100.75 109.9) (width 0.2) (layer "B.Cu") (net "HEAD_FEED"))
 (segment (start 100 109.375) (end 100.45 109.825) (width 0.2) (layer "B.Cu") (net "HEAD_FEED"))
 (segment (start 102.4 107.125) (end 102.4 107.05) (width 0.2) (layer "B.Cu") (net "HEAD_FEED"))
 (segment (start 102.25 107.2) (end 102.325 107.2) (width 0.2) (layer "B.Cu") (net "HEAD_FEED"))
 (segment (start 98.275 99.4) (end 98.275 99.325) (width 0.2) (layer "B.Cu") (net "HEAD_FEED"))
 (segment (start 99.1 109.975) (end 99.4 109.675) (width 0.2) (layer "B.Cu") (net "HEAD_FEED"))
 (segment (start 102.55 102.55) (end 102.7 102.4) (width 0.2) (layer "B.Cu") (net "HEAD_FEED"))
 (segment (start 101.425 109.75) (end 101.425 109.675) (width 0.2) (layer "B.Cu") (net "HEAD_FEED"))
 (segment (start 97.3 100.375) (end 98.275 99.4) (width 0.2) (layer "B.Cu") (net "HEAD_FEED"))
 (segment (start 102.025 107.275) (end 102.175 107.275) (width 0.2) (layer "B.Cu") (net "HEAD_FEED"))
 (segment (start 102.85 102.1) (end 102.85 98.8) (width 0.2) (layer "B.Cu") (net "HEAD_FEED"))
 (segment (start 101.2 109.975) (end 101.425 109.75) (width 0.2) (layer "B.Cu") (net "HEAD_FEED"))
 (segment (start 101.95 107.35) (end 102.025 107.275) (width 0.2) (layer "B.Cu") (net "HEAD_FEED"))
 (segment (start 102.175 107.275) (end 102.25 107.2) (width 0.2) (layer "B.Cu") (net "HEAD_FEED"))
 (segment (start 102.325 107.2) (end 102.4 107.125) (width 0.2) (layer "B.Cu") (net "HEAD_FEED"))
 (segment (start 101.575 109.375) (end 101.575 107.8) (width 0.2) (layer "B.Cu") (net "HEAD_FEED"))
 (segment (start 100.525 109.825) (end 100.6 109.9) (width 0.2) (layer "B.Cu") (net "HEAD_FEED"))
 (segment (start 100.825 109.975) (end 101.2 109.975) (width 0.2) (layer "B.Cu") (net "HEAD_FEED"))
 (segment (start 100.75 102.175) (end 100.675 102.25) (width 0.2) (layer "F.Cu") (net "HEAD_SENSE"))
 (segment (start 102.775 101.275) (end 103.25 100.875) (width 0.2) (layer "F.Cu") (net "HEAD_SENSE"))
 (segment (start 101.875 106.975) (end 101.875 106.675) (width 0.2) (layer "F.Cu") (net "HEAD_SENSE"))
 (segment (start 101.875 102.175) (end 100.75 102.175) (width 0.2) (layer "F.Cu") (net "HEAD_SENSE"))
 (segment (start 98.65 102.25) (end 97.3 103.6) (width 0.2) (layer "F.Cu") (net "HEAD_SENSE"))
 (segment (start 100.675 102.25) (end 98.65 102.25) (width 0.2) (layer "F.Cu") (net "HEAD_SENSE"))
 (segment (start 101.875 106.975) (end 101.875 106.675) (width 0.2) (layer "F.Cu") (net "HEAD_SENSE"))
 (segment (start 97.3 103.6) (end 96.8 104.025) (width 0.2) (layer "F.Cu") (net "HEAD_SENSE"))
 (segment (start 102.775 101.275) (end 101.875 102.175) (width 0.2) (layer "F.Cu") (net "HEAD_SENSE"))
 (via (at 101.875 106.675) (size 0.6) (drill 0.3) (layers "F.Cu" "B.Cu") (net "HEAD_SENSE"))
 (via (at 101.875 102.325) (size 0.6) (drill 0.3) (layers "F.Cu" "B.Cu") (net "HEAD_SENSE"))
 (segment (start 101.875 106.675) (end 101.875 102.325) (width 0.2) (layer "B.Cu") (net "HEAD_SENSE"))
 (segment (start 100.3 105.4) (end 100 105.7) (width 0.2) (layer "F.Cu") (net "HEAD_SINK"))
 (segment (start 100.3 105.325) (end 100.3 105.4) (width 0.2) (layer "F.Cu") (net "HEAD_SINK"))
 (segment (start 98.125 106) (end 97.6 106) (width 0.2) (layer "F.Cu") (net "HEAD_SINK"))
 (segment (start 97.225 106.375) (end 96.965 106.615) (width 0.2) (layer "F.Cu") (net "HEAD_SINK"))
 (segment (start 97.6 106) (end 97.225 106.375) (width 0.2) (layer "F.Cu") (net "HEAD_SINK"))
 (segment (start 102.775 105.4) (end 103.25 105.825) (width 0.2) (layer "F.Cu") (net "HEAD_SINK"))
 (segment (start 100.375 105.25) (end 100.3 105.325) (width 0.2) (layer "F.Cu") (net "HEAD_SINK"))
 (segment (start 98.5 109.9) (end 99.2125 110.225) (width 0.2) (layer "F.Cu") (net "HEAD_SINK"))
 (segment (start 98.05 107.8) (end 96.965 106.615) (width 0.2) (layer "F.Cu") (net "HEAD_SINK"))
 (segment (start 101.8 105.1) (end 100.45 105.1) (width 0.2) (layer "F.Cu") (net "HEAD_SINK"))
 (segment (start 98.5 109.9) (end 98.35 109.9) (width 0.2) (layer "F.Cu") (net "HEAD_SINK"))
 (segment (start 98.2 109.15) (end 98.05 109) (width 0.2) (layer "F.Cu") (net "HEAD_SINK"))
 (segment (start 98.35 109.9) (end 98.2 109.75) (width 0.2) (layer "F.Cu") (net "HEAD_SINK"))
 (segment (start 102.775 105.4) (end 102.1 105.4) (width 0.2) (layer "F.Cu") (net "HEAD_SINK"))
 (segment (start 100.45 105.1) (end 100.375 105.175) (width 0.2) (layer "F.Cu") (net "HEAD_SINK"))
 (segment (start 102.1 105.4) (end 101.8 105.1) (width 0.2) (layer "F.Cu") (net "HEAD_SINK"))
 (segment (start 98.425 105.7) (end 98.125 106) (width 0.2) (layer "F.Cu") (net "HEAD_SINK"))
 (segment (start 98.05 109) (end 98.05 107.8) (width 0.2) (layer "F.Cu") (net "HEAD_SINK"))
 (segment (start 100.375 105.175) (end 100.375 105.25) (width 0.2) (layer "F.Cu") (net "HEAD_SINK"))
 (segment (start 100 105.7) (end 98.425 105.7) (width 0.2) (layer "F.Cu") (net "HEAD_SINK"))
 (segment (start 98.2 109.75) (end 98.2 109.15) (width 0.2) (layer "F.Cu") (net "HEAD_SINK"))
 (via (at 99.55 108.4) (size 0.6) (drill 0.3) (layers "F.Cu" "B.Cu") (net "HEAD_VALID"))
 (via (at 100.9 109.3) (size 0.6) (drill 0.3) (layers "F.Cu" "B.Cu") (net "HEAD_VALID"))
 (via (at 100.675 104.425) (size 0.6) (drill 0.3) (layers "F.Cu" "B.Cu") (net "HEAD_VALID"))
 (segment (start 99.925 108.625) (end 99.775 108.625) (width 0.2) (layer "B.Cu") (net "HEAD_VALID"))
 (segment (start 100.6 109.3) (end 99.925 108.625) (width 0.2) (layer "B.Cu") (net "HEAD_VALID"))
 (segment (start 100.675 107.125) (end 99.7 108.1) (width 0.2) (layer "B.Cu") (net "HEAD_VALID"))
 (segment (start 99.775 108.625) (end 99.55 108.4) (width 0.2) (layer "B.Cu") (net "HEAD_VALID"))
 (segment (start 100.675 104.425) (end 100.675 107.125) (width 0.2) (layer "B.Cu") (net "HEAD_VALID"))
 (segment (start 100.9 109.3) (end 100.6 109.3) (width 0.2) (layer "B.Cu") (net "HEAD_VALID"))
 (segment (start 100.225 111.325) (end 100.225 107.35) (width 0.2) (layer "F.Cu") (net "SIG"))
 (segment (start 100.225 107.35) (end 99.85 106.975) (width 0.2) (layer "F.Cu") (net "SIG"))
 (segment (start 99.85 106.975) (end 99.35 106.575) (width 0.2) (layer "F.Cu") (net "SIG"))
 (segment (start 100.225 111.325) (end 100 112.25) (width 0.2) (layer "F.Cu") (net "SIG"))
 (segment (start 98.875 105.25) (end 99.35 104.925) (width 0.2) (layer "F.Cu") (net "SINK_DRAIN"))
 (segment (start 97.465 105.325) (end 98.875 105.25) (width 0.2) (layer "F.Cu") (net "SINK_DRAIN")))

